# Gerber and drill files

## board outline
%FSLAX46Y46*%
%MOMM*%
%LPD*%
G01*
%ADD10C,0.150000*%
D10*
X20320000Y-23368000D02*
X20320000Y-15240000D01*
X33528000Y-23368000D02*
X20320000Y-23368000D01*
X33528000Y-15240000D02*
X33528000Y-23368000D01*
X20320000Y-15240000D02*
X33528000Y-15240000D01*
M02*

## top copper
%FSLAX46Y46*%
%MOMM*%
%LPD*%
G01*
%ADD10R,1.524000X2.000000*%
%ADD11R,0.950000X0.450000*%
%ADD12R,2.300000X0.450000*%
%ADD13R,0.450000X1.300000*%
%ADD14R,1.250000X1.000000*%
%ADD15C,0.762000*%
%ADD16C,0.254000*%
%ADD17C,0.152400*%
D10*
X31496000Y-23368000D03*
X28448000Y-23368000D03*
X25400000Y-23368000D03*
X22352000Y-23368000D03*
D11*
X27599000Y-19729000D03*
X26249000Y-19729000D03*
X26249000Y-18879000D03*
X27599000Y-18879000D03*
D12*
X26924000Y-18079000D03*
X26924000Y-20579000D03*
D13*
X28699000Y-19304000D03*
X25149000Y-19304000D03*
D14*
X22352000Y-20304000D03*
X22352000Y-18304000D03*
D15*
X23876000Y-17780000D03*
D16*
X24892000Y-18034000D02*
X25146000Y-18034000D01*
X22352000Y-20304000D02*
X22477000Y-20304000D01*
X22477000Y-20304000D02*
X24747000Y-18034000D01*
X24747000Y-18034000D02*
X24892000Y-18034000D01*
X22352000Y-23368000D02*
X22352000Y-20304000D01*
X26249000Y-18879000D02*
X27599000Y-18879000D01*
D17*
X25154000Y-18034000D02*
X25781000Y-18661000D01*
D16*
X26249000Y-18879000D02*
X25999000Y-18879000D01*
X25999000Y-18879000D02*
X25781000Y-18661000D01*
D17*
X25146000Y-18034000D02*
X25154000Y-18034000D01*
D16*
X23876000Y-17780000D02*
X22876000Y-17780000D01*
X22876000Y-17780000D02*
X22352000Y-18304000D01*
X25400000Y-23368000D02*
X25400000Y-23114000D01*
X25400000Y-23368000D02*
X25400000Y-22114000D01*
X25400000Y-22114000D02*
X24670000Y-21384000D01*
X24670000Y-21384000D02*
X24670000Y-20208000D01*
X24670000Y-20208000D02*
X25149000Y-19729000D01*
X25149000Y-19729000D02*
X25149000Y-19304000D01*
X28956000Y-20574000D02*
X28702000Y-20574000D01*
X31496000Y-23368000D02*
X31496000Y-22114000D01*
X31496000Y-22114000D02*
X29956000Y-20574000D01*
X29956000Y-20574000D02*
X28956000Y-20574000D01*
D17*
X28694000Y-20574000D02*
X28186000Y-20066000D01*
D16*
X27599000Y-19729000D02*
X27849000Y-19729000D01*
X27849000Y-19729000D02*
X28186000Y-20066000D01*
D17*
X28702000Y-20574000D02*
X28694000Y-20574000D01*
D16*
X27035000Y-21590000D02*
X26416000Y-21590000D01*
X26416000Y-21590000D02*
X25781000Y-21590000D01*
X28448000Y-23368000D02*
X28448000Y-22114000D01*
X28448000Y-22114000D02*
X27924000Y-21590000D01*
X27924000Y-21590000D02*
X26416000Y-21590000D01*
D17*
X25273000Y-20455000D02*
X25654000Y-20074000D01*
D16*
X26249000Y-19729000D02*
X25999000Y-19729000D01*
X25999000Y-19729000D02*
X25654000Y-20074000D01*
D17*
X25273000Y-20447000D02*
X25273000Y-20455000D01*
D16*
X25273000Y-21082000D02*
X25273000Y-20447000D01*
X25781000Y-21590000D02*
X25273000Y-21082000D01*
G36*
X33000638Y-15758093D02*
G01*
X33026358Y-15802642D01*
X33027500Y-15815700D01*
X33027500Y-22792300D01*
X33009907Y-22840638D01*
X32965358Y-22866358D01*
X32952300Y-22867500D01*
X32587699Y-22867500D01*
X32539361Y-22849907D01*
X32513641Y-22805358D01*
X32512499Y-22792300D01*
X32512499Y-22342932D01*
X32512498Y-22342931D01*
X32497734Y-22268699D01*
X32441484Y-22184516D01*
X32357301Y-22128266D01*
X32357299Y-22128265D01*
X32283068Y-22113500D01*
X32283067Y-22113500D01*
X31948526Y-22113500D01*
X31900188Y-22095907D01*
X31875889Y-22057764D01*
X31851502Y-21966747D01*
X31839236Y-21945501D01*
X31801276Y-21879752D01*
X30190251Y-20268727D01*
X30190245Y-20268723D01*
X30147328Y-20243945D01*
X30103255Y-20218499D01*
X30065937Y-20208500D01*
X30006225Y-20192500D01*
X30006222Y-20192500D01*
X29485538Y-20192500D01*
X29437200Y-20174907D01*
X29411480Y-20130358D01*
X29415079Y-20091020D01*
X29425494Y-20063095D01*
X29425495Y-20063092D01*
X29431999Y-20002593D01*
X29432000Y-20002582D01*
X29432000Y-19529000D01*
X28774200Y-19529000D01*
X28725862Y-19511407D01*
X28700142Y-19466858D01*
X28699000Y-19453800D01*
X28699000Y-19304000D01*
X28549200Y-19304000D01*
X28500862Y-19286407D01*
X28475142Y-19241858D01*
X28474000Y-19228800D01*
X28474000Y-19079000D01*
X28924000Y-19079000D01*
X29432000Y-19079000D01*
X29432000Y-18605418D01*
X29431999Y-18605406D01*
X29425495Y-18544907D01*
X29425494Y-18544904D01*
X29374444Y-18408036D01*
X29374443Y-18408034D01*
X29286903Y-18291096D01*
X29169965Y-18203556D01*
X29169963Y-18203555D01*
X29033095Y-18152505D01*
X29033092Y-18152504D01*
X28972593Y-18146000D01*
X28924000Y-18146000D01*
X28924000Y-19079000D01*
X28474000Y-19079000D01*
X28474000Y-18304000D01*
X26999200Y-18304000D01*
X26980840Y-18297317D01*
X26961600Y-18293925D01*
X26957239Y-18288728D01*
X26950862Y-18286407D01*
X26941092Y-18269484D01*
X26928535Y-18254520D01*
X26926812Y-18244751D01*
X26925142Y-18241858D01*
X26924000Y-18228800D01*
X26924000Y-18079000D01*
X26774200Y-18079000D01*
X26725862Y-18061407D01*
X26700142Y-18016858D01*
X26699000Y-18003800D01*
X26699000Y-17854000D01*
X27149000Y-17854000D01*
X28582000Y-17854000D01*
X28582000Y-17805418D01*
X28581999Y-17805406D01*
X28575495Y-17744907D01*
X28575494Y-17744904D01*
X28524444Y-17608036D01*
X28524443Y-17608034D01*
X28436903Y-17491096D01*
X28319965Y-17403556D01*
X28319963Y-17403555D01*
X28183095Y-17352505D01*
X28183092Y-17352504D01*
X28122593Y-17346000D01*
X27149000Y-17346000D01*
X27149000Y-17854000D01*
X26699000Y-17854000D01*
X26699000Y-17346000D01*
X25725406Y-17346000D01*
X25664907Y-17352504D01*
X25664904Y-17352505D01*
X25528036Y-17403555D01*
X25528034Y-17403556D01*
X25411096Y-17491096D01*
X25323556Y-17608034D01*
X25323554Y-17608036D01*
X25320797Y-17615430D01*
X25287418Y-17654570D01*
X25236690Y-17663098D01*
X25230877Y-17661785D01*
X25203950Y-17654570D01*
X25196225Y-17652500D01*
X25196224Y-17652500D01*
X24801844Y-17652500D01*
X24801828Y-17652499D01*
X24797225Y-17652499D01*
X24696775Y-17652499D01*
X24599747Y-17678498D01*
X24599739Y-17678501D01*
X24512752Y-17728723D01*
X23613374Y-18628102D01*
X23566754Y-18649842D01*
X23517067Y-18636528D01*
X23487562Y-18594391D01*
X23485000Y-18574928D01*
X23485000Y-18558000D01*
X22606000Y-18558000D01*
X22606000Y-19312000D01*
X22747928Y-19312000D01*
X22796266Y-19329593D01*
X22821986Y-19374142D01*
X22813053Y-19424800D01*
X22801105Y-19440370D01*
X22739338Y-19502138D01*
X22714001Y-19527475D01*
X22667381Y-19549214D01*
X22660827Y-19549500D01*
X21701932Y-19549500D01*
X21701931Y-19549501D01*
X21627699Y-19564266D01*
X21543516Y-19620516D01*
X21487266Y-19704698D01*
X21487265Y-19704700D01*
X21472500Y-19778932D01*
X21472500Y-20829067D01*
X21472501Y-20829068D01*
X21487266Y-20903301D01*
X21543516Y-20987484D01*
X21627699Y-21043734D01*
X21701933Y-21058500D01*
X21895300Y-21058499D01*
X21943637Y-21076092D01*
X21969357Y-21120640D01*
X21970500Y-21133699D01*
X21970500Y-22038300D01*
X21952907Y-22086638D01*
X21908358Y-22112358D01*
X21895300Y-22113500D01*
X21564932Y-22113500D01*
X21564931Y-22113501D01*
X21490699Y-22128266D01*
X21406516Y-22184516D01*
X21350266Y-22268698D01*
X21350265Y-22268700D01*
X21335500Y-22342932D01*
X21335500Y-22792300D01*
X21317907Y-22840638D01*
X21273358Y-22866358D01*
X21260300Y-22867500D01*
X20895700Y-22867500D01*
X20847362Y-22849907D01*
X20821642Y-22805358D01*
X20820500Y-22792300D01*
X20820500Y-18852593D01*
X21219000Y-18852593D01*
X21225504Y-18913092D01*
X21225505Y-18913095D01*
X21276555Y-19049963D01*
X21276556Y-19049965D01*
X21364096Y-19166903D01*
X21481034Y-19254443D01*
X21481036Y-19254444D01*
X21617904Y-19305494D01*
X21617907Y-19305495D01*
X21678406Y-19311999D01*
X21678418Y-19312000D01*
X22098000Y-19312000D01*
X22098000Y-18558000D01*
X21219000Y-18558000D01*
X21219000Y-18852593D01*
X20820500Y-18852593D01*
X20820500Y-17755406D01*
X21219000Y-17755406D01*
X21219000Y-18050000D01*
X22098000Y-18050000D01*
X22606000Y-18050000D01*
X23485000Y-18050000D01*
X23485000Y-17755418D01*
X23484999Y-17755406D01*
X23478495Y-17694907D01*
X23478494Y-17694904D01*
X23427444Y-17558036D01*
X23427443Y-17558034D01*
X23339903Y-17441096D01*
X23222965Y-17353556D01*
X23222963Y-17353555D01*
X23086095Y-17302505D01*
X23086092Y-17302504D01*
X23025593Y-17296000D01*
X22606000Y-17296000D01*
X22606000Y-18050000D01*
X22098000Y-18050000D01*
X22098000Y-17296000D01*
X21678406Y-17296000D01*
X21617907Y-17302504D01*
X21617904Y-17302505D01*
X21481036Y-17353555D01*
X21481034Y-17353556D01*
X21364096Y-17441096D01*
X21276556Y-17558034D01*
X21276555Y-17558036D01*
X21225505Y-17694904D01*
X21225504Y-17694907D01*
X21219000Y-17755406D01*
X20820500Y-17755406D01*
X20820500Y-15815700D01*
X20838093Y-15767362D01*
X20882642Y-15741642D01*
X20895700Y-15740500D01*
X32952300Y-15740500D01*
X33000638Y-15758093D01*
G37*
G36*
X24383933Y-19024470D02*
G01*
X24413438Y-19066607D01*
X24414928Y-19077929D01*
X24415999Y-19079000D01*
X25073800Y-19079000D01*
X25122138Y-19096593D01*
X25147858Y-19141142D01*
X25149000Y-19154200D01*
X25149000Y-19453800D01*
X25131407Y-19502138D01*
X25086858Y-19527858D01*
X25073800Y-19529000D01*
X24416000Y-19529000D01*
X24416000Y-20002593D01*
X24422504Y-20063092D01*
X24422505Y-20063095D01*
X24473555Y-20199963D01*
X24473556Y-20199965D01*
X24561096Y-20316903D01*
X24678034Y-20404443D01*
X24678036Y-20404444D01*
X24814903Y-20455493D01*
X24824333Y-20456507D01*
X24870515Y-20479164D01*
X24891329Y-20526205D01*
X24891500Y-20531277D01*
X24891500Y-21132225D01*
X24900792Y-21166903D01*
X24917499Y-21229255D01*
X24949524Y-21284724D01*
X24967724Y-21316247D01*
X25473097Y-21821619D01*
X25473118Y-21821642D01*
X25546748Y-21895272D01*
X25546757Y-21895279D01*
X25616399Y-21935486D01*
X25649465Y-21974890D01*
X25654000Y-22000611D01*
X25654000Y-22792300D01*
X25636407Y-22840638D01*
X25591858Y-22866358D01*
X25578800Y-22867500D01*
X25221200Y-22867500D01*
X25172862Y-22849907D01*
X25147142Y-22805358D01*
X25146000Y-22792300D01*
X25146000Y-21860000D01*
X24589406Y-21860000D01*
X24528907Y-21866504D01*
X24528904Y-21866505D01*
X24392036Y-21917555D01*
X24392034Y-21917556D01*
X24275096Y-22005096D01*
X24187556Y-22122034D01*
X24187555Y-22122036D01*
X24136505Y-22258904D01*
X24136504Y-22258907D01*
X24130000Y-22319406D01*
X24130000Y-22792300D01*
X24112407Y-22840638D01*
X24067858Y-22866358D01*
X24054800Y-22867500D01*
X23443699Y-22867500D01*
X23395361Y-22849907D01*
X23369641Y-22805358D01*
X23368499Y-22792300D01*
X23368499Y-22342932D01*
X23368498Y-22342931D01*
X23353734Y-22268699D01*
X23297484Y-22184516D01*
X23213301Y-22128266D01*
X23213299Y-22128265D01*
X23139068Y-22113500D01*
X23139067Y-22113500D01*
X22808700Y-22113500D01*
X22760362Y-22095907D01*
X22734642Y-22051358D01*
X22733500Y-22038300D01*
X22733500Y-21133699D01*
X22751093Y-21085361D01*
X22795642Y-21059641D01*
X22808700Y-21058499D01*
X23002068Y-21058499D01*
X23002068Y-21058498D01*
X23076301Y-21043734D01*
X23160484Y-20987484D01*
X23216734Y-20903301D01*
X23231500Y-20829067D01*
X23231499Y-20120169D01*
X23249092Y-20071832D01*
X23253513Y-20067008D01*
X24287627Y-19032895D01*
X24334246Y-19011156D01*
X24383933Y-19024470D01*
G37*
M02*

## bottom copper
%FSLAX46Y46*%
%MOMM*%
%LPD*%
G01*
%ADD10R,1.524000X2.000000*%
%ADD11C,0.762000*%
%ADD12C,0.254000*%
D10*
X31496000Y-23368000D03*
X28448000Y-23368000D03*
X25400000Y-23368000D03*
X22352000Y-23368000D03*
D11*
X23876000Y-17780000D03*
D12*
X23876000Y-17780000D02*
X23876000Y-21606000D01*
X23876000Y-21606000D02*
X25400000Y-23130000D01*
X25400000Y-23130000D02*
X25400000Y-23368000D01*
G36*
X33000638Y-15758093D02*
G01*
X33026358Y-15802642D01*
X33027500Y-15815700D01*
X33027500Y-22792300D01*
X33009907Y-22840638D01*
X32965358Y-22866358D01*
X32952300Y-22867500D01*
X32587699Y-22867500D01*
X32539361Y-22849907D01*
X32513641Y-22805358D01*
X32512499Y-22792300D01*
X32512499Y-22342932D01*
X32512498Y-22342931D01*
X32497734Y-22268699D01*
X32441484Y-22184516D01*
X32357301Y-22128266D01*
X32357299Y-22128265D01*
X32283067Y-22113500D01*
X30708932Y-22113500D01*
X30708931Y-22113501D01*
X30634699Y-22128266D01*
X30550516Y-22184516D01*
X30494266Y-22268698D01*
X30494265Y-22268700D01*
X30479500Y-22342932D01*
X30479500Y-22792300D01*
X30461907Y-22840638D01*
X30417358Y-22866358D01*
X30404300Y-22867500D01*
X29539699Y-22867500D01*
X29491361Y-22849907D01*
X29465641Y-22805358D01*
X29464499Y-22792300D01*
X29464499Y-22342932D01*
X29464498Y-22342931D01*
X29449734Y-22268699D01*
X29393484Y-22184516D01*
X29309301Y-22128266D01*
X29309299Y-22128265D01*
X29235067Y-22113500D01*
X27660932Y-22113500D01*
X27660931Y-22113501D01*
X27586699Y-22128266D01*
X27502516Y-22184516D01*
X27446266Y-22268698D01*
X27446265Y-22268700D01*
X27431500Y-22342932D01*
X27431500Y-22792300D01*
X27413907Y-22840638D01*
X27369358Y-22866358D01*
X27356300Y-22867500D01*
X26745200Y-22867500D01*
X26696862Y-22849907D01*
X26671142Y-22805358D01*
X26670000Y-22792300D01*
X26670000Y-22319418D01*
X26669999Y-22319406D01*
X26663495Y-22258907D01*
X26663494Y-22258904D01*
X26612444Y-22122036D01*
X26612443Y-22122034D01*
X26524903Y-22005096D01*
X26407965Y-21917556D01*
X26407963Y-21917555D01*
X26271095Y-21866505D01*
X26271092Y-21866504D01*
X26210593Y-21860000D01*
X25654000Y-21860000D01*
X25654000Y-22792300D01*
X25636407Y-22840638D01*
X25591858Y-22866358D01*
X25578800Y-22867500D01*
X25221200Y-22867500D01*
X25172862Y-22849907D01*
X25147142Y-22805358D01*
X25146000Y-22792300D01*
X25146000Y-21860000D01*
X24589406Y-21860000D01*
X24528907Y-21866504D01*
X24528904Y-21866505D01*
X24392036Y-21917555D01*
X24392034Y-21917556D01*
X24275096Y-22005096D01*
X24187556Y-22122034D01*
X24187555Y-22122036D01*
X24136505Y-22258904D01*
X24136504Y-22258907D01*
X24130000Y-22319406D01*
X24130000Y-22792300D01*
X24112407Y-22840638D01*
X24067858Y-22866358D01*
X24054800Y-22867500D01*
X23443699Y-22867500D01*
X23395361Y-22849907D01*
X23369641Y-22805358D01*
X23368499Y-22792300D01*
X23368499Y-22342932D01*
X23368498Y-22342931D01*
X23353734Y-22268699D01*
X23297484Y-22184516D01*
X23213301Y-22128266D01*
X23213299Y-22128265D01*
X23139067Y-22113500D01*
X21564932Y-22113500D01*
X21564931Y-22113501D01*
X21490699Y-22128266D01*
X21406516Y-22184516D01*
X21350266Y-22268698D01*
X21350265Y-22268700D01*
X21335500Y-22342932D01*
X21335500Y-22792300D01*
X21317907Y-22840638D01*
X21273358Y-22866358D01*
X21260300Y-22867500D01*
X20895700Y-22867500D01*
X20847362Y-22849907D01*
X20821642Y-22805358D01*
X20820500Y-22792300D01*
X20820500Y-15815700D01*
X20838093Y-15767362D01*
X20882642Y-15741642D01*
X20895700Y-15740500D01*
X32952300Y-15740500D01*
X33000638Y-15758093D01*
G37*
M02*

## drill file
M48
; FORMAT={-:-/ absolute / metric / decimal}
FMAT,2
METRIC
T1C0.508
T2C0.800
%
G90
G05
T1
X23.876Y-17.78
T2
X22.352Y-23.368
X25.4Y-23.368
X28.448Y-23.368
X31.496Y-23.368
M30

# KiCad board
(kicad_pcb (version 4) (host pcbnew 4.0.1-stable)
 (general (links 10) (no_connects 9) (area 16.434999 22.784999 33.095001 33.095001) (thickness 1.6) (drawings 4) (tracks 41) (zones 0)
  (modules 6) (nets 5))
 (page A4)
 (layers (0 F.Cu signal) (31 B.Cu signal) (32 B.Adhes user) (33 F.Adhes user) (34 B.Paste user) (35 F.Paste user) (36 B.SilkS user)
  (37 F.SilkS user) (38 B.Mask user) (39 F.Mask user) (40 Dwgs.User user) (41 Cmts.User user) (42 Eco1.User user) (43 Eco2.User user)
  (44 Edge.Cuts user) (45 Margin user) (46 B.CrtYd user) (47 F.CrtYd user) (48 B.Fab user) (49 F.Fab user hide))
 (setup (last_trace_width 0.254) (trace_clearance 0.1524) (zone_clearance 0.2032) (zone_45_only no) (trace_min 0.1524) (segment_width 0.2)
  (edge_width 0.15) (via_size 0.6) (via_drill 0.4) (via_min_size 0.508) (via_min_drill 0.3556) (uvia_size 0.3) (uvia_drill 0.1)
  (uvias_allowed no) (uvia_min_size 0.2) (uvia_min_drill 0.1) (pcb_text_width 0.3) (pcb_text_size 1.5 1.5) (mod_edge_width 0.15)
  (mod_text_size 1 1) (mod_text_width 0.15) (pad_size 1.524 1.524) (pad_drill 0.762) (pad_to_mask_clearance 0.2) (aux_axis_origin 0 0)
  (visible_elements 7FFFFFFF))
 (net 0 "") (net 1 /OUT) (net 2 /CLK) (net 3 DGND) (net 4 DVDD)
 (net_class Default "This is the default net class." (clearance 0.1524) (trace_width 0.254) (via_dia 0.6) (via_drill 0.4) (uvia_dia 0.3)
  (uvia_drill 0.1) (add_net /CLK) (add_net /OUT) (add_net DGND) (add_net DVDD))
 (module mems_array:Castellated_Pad (layer F.Cu) (at 31.496 23.368)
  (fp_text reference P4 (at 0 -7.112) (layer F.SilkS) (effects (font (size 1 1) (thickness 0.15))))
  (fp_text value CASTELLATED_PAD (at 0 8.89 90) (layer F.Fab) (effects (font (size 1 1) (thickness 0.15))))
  (pad 1 thru_hole rect (at 0 0) (size 1.524 2) (drill 0.8) (layers *.Cu *.Mask F.SilkS) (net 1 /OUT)))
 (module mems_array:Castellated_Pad (layer F.Cu) (at 28.448 23.368)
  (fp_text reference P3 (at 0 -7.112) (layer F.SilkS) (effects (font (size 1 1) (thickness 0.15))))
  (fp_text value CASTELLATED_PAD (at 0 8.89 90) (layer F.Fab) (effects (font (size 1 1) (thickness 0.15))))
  (pad 1 thru_hole rect (at 0 0) (size 1.524 2) (drill 0.8) (layers *.Cu *.Mask F.SilkS) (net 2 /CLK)))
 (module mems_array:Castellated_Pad (layer F.Cu) (at 25.4 23.368)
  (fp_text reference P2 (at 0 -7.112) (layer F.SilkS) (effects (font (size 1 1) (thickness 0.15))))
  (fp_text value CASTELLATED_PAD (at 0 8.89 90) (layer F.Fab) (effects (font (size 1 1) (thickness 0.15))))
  (pad 1 thru_hole rect (at 0 0) (size 1.524 2) (drill 0.8) (layers *.Cu *.Mask F.SilkS) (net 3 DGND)))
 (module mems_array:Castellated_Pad (layer F.Cu) (at 22.352 23.368)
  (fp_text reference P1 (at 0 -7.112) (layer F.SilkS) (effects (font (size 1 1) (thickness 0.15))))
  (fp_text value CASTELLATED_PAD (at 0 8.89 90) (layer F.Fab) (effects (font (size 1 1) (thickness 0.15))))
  (pad 1 thru_hole rect (at 0 0) (size 1.524 2) (drill 0.8) (layers *.Cu *.Mask F.SilkS) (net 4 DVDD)))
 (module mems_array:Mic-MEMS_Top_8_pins (layer F.Cu) (at 26.924 19.304 90)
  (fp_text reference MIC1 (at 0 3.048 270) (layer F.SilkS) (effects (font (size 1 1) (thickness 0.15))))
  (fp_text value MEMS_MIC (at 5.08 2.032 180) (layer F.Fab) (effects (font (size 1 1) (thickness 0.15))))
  (pad 4 smd rect (at -0.425 0.675 90) (size 0.45 0.95) (layers F.Cu F.Paste F.Mask) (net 1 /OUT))
  (pad 3 smd rect (at -0.425 -0.675 90) (size 0.45 0.95) (layers F.Cu F.Paste F.Mask) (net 2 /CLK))
  (pad 2 smd rect (at 0.425 -0.675 90) (size 0.45 0.95) (layers F.Cu F.Paste F.Mask) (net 4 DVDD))
  (pad 1 smd rect (at 0.425 0.675 90) (size 0.45 0.95) (layers F.Cu F.Paste F.Mask) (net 4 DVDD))
  (pad 5 smd rect (at 1.225 0 90) (size 0.45 2.3) (layers F.Cu F.Paste F.Mask) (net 3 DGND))
  (pad 5 smd rect (at -1.275 0 90) (size 0.45 2.3) (layers F.Cu F.Paste F.Mask) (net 3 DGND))
  (pad 5 smd rect (at 0 1.775 90) (size 1.3 0.45) (layers F.Cu F.Paste F.Mask) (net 3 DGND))
  (pad 5 smd rect (at 0 -1.775 90) (size 1.3 0.45) (layers F.Cu F.Paste F.Mask) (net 3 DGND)))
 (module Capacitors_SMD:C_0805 (layer F.Cu) (at 22.352 19.304 90)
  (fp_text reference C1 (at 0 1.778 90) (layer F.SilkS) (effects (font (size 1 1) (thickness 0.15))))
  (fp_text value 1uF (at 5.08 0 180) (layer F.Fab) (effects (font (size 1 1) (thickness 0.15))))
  (pad 1 smd rect (at -1 0 90) (size 1 1.25) (layers F.Cu F.Paste F.Mask) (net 4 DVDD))
  (pad 2 smd rect (at 1 0 90) (size 1 1.25) (layers F.Cu F.Paste F.Mask) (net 3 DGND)))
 (gr_line (start 20.32 23.368) (end 20.32 15.24) (layer Edge.Cuts) (width 0.15))
 (gr_line (start 33.528 23.368) (end 20.32 23.368) (layer Edge.Cuts) (width 0.15))
 (gr_line (start 33.528 15.24) (end 33.528 23.368) (layer Edge.Cuts) (width 0.15))
 (gr_line (start 20.32 15.24) (end 33.528 15.24) (layer Edge.Cuts) (width 0.15))
 (segment (start 24.892 18.034) (end 25.146 18.034) (width 0.254) (layer F.Cu) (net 4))
 (segment (start 22.352 20.304) (end 22.477 20.304) (width 0.254) (layer F.Cu) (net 4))
 (segment (start 22.477 20.304) (end 24.747 18.034) (width 0.254) (layer F.Cu) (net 4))
 (segment (start 24.747 18.034) (end 24.892 18.034) (width 0.254) (layer F.Cu) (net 4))
 (segment (start 22.352 23.368) (end 22.352 20.304) (width 0.254) (layer F.Cu) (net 4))
 (segment (start 26.249 18.879) (end 27.599 18.879) (width 0.254) (layer F.Cu) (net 4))
 (segment (start 25.154 18.034) (end 25.781 18.661) (width 0.1524) (layer F.Cu) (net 4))
 (segment (start 26.249 18.879) (end 25.999 18.879) (width 0.254) (layer F.Cu) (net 4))
 (segment (start 25.999 18.879) (end 25.781 18.661) (width 0.254) (layer F.Cu) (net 4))
 (segment (start 25.146 18.034) (end 25.154 18.034) (width 0.1524) (layer F.Cu) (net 4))
 (segment (start 23.876 17.78) (end 23.876 21.606) (width 0.254) (layer B.Cu) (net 3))
 (segment (start 23.876 21.606) (end 25.4 23.13) (width 0.254) (layer B.Cu) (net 3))
 (segment (start 25.4 23.13) (end 25.4 23.368) (width 0.254) (layer B.Cu) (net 3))
 (segment (start 23.876 17.78) (end 22.876 17.78) (width 0.254) (layer F.Cu) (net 3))
 (segment (start 22.876 17.78) (end 22.352 18.304) (width 0.254) (layer F.Cu) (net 3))
 (via (at 23.876 17.78) (size 0.762) (drill 0.508) (layers F.Cu B.Cu) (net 3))
 (segment (start 25.4 23.368) (end 25.4 23.114) (width 0.254) (layer F.Cu) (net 3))
 (segment (start 25.4 23.368) (end 25.4 22.114) (width 0.254) (layer F.Cu) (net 3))
 (segment (start 25.4 22.114) (end 24.67 21.384) (width 0.254) (layer F.Cu) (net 3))
 (segment (start 24.67 21.384) (end 24.67 20.208) (width 0.254) (layer F.Cu) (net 3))
 (segment (start 24.67 20.208) (end 25.149 19.729) (width 0.254) (layer F.Cu) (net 3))
 (segment (start 25.149 19.729) (end 25.149 19.304) (width 0.254) (layer F.Cu) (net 3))
 (segment (start 28.956 20.574) (end 28.702 20.574) (width 0.254) (layer F.Cu) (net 1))
 (segment (start 31.496 23.368) (end 31.496 22.114) (width 0.254) (layer F.Cu) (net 1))
 (segment (start 31.496 22.114) (end 29.956 20.574) (width 0.254) (layer F.Cu) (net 1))
 (segment (start 29.956 20.574) (end 28.956 20.574) (width 0.254) (layer F.Cu) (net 1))
 (segment (start 28.694 20.574) (end 28.186 20.066) (width 0.1524) (layer F.Cu) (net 1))
 (segment (start 27.599 19.729) (end 27.849 19.729) (width 0.254) (layer F.Cu) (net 1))
 (segment (start 27.849 19.729) (end 28.186 20.066) (width 0.254) (layer F.Cu) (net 1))
 (segment (start 28.702 20.574) (end 28.694 20.574) (width 0.1524) (layer F.Cu) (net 1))
 (segment (start 27.035 21.59) (end 26.416 21.59) (width 0.254) (layer F.Cu) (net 2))
 (segment (start 26.416 21.59) (end 25.781 21.59) (width 0.254) (layer F.Cu) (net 2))
 (segment (start 28.448 23.368) (end 28.448 22.114) (width 0.254) (layer F.Cu) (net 2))
 (segment (start 28.448 22.114) (end 27.924 21.59) (width 0.254) (layer F.Cu) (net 2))
 (segment (start 27.924 21.59) (end 26.416 21.59) (width 0.254) (layer F.Cu) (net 2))
 (segment (start 25.273 20.455) (end 25.654 20.074) (width 0.1524) (layer F.Cu) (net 2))
 (segment (start 26.249 19.729) (end 25.999 19.729) (width 0.254) (layer F.Cu) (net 2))
 (segment (start 25.999 19.729) (end 25.654 20.074) (width 0.254) (layer F.Cu) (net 2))
 (segment (start 25.273 20.447) (end 25.273 20.455) (width 0.1524) (layer F.Cu) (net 2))
 (segment (start 25.273 21.082) (end 25.273 20.447) (width 0.254) (layer F.Cu) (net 2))
 (segment (start 25.781 21.59) (end 25.273 21.082) (width 0.254) (layer F.Cu) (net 2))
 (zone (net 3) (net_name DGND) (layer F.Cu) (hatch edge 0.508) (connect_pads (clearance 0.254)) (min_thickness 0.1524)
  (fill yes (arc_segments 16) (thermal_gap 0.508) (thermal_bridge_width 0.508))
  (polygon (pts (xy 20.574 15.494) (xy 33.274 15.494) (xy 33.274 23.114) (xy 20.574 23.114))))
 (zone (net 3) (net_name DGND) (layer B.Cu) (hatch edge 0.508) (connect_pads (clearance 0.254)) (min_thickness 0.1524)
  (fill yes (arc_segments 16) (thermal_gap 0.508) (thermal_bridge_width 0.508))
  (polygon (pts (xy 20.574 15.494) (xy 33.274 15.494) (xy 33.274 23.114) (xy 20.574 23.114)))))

